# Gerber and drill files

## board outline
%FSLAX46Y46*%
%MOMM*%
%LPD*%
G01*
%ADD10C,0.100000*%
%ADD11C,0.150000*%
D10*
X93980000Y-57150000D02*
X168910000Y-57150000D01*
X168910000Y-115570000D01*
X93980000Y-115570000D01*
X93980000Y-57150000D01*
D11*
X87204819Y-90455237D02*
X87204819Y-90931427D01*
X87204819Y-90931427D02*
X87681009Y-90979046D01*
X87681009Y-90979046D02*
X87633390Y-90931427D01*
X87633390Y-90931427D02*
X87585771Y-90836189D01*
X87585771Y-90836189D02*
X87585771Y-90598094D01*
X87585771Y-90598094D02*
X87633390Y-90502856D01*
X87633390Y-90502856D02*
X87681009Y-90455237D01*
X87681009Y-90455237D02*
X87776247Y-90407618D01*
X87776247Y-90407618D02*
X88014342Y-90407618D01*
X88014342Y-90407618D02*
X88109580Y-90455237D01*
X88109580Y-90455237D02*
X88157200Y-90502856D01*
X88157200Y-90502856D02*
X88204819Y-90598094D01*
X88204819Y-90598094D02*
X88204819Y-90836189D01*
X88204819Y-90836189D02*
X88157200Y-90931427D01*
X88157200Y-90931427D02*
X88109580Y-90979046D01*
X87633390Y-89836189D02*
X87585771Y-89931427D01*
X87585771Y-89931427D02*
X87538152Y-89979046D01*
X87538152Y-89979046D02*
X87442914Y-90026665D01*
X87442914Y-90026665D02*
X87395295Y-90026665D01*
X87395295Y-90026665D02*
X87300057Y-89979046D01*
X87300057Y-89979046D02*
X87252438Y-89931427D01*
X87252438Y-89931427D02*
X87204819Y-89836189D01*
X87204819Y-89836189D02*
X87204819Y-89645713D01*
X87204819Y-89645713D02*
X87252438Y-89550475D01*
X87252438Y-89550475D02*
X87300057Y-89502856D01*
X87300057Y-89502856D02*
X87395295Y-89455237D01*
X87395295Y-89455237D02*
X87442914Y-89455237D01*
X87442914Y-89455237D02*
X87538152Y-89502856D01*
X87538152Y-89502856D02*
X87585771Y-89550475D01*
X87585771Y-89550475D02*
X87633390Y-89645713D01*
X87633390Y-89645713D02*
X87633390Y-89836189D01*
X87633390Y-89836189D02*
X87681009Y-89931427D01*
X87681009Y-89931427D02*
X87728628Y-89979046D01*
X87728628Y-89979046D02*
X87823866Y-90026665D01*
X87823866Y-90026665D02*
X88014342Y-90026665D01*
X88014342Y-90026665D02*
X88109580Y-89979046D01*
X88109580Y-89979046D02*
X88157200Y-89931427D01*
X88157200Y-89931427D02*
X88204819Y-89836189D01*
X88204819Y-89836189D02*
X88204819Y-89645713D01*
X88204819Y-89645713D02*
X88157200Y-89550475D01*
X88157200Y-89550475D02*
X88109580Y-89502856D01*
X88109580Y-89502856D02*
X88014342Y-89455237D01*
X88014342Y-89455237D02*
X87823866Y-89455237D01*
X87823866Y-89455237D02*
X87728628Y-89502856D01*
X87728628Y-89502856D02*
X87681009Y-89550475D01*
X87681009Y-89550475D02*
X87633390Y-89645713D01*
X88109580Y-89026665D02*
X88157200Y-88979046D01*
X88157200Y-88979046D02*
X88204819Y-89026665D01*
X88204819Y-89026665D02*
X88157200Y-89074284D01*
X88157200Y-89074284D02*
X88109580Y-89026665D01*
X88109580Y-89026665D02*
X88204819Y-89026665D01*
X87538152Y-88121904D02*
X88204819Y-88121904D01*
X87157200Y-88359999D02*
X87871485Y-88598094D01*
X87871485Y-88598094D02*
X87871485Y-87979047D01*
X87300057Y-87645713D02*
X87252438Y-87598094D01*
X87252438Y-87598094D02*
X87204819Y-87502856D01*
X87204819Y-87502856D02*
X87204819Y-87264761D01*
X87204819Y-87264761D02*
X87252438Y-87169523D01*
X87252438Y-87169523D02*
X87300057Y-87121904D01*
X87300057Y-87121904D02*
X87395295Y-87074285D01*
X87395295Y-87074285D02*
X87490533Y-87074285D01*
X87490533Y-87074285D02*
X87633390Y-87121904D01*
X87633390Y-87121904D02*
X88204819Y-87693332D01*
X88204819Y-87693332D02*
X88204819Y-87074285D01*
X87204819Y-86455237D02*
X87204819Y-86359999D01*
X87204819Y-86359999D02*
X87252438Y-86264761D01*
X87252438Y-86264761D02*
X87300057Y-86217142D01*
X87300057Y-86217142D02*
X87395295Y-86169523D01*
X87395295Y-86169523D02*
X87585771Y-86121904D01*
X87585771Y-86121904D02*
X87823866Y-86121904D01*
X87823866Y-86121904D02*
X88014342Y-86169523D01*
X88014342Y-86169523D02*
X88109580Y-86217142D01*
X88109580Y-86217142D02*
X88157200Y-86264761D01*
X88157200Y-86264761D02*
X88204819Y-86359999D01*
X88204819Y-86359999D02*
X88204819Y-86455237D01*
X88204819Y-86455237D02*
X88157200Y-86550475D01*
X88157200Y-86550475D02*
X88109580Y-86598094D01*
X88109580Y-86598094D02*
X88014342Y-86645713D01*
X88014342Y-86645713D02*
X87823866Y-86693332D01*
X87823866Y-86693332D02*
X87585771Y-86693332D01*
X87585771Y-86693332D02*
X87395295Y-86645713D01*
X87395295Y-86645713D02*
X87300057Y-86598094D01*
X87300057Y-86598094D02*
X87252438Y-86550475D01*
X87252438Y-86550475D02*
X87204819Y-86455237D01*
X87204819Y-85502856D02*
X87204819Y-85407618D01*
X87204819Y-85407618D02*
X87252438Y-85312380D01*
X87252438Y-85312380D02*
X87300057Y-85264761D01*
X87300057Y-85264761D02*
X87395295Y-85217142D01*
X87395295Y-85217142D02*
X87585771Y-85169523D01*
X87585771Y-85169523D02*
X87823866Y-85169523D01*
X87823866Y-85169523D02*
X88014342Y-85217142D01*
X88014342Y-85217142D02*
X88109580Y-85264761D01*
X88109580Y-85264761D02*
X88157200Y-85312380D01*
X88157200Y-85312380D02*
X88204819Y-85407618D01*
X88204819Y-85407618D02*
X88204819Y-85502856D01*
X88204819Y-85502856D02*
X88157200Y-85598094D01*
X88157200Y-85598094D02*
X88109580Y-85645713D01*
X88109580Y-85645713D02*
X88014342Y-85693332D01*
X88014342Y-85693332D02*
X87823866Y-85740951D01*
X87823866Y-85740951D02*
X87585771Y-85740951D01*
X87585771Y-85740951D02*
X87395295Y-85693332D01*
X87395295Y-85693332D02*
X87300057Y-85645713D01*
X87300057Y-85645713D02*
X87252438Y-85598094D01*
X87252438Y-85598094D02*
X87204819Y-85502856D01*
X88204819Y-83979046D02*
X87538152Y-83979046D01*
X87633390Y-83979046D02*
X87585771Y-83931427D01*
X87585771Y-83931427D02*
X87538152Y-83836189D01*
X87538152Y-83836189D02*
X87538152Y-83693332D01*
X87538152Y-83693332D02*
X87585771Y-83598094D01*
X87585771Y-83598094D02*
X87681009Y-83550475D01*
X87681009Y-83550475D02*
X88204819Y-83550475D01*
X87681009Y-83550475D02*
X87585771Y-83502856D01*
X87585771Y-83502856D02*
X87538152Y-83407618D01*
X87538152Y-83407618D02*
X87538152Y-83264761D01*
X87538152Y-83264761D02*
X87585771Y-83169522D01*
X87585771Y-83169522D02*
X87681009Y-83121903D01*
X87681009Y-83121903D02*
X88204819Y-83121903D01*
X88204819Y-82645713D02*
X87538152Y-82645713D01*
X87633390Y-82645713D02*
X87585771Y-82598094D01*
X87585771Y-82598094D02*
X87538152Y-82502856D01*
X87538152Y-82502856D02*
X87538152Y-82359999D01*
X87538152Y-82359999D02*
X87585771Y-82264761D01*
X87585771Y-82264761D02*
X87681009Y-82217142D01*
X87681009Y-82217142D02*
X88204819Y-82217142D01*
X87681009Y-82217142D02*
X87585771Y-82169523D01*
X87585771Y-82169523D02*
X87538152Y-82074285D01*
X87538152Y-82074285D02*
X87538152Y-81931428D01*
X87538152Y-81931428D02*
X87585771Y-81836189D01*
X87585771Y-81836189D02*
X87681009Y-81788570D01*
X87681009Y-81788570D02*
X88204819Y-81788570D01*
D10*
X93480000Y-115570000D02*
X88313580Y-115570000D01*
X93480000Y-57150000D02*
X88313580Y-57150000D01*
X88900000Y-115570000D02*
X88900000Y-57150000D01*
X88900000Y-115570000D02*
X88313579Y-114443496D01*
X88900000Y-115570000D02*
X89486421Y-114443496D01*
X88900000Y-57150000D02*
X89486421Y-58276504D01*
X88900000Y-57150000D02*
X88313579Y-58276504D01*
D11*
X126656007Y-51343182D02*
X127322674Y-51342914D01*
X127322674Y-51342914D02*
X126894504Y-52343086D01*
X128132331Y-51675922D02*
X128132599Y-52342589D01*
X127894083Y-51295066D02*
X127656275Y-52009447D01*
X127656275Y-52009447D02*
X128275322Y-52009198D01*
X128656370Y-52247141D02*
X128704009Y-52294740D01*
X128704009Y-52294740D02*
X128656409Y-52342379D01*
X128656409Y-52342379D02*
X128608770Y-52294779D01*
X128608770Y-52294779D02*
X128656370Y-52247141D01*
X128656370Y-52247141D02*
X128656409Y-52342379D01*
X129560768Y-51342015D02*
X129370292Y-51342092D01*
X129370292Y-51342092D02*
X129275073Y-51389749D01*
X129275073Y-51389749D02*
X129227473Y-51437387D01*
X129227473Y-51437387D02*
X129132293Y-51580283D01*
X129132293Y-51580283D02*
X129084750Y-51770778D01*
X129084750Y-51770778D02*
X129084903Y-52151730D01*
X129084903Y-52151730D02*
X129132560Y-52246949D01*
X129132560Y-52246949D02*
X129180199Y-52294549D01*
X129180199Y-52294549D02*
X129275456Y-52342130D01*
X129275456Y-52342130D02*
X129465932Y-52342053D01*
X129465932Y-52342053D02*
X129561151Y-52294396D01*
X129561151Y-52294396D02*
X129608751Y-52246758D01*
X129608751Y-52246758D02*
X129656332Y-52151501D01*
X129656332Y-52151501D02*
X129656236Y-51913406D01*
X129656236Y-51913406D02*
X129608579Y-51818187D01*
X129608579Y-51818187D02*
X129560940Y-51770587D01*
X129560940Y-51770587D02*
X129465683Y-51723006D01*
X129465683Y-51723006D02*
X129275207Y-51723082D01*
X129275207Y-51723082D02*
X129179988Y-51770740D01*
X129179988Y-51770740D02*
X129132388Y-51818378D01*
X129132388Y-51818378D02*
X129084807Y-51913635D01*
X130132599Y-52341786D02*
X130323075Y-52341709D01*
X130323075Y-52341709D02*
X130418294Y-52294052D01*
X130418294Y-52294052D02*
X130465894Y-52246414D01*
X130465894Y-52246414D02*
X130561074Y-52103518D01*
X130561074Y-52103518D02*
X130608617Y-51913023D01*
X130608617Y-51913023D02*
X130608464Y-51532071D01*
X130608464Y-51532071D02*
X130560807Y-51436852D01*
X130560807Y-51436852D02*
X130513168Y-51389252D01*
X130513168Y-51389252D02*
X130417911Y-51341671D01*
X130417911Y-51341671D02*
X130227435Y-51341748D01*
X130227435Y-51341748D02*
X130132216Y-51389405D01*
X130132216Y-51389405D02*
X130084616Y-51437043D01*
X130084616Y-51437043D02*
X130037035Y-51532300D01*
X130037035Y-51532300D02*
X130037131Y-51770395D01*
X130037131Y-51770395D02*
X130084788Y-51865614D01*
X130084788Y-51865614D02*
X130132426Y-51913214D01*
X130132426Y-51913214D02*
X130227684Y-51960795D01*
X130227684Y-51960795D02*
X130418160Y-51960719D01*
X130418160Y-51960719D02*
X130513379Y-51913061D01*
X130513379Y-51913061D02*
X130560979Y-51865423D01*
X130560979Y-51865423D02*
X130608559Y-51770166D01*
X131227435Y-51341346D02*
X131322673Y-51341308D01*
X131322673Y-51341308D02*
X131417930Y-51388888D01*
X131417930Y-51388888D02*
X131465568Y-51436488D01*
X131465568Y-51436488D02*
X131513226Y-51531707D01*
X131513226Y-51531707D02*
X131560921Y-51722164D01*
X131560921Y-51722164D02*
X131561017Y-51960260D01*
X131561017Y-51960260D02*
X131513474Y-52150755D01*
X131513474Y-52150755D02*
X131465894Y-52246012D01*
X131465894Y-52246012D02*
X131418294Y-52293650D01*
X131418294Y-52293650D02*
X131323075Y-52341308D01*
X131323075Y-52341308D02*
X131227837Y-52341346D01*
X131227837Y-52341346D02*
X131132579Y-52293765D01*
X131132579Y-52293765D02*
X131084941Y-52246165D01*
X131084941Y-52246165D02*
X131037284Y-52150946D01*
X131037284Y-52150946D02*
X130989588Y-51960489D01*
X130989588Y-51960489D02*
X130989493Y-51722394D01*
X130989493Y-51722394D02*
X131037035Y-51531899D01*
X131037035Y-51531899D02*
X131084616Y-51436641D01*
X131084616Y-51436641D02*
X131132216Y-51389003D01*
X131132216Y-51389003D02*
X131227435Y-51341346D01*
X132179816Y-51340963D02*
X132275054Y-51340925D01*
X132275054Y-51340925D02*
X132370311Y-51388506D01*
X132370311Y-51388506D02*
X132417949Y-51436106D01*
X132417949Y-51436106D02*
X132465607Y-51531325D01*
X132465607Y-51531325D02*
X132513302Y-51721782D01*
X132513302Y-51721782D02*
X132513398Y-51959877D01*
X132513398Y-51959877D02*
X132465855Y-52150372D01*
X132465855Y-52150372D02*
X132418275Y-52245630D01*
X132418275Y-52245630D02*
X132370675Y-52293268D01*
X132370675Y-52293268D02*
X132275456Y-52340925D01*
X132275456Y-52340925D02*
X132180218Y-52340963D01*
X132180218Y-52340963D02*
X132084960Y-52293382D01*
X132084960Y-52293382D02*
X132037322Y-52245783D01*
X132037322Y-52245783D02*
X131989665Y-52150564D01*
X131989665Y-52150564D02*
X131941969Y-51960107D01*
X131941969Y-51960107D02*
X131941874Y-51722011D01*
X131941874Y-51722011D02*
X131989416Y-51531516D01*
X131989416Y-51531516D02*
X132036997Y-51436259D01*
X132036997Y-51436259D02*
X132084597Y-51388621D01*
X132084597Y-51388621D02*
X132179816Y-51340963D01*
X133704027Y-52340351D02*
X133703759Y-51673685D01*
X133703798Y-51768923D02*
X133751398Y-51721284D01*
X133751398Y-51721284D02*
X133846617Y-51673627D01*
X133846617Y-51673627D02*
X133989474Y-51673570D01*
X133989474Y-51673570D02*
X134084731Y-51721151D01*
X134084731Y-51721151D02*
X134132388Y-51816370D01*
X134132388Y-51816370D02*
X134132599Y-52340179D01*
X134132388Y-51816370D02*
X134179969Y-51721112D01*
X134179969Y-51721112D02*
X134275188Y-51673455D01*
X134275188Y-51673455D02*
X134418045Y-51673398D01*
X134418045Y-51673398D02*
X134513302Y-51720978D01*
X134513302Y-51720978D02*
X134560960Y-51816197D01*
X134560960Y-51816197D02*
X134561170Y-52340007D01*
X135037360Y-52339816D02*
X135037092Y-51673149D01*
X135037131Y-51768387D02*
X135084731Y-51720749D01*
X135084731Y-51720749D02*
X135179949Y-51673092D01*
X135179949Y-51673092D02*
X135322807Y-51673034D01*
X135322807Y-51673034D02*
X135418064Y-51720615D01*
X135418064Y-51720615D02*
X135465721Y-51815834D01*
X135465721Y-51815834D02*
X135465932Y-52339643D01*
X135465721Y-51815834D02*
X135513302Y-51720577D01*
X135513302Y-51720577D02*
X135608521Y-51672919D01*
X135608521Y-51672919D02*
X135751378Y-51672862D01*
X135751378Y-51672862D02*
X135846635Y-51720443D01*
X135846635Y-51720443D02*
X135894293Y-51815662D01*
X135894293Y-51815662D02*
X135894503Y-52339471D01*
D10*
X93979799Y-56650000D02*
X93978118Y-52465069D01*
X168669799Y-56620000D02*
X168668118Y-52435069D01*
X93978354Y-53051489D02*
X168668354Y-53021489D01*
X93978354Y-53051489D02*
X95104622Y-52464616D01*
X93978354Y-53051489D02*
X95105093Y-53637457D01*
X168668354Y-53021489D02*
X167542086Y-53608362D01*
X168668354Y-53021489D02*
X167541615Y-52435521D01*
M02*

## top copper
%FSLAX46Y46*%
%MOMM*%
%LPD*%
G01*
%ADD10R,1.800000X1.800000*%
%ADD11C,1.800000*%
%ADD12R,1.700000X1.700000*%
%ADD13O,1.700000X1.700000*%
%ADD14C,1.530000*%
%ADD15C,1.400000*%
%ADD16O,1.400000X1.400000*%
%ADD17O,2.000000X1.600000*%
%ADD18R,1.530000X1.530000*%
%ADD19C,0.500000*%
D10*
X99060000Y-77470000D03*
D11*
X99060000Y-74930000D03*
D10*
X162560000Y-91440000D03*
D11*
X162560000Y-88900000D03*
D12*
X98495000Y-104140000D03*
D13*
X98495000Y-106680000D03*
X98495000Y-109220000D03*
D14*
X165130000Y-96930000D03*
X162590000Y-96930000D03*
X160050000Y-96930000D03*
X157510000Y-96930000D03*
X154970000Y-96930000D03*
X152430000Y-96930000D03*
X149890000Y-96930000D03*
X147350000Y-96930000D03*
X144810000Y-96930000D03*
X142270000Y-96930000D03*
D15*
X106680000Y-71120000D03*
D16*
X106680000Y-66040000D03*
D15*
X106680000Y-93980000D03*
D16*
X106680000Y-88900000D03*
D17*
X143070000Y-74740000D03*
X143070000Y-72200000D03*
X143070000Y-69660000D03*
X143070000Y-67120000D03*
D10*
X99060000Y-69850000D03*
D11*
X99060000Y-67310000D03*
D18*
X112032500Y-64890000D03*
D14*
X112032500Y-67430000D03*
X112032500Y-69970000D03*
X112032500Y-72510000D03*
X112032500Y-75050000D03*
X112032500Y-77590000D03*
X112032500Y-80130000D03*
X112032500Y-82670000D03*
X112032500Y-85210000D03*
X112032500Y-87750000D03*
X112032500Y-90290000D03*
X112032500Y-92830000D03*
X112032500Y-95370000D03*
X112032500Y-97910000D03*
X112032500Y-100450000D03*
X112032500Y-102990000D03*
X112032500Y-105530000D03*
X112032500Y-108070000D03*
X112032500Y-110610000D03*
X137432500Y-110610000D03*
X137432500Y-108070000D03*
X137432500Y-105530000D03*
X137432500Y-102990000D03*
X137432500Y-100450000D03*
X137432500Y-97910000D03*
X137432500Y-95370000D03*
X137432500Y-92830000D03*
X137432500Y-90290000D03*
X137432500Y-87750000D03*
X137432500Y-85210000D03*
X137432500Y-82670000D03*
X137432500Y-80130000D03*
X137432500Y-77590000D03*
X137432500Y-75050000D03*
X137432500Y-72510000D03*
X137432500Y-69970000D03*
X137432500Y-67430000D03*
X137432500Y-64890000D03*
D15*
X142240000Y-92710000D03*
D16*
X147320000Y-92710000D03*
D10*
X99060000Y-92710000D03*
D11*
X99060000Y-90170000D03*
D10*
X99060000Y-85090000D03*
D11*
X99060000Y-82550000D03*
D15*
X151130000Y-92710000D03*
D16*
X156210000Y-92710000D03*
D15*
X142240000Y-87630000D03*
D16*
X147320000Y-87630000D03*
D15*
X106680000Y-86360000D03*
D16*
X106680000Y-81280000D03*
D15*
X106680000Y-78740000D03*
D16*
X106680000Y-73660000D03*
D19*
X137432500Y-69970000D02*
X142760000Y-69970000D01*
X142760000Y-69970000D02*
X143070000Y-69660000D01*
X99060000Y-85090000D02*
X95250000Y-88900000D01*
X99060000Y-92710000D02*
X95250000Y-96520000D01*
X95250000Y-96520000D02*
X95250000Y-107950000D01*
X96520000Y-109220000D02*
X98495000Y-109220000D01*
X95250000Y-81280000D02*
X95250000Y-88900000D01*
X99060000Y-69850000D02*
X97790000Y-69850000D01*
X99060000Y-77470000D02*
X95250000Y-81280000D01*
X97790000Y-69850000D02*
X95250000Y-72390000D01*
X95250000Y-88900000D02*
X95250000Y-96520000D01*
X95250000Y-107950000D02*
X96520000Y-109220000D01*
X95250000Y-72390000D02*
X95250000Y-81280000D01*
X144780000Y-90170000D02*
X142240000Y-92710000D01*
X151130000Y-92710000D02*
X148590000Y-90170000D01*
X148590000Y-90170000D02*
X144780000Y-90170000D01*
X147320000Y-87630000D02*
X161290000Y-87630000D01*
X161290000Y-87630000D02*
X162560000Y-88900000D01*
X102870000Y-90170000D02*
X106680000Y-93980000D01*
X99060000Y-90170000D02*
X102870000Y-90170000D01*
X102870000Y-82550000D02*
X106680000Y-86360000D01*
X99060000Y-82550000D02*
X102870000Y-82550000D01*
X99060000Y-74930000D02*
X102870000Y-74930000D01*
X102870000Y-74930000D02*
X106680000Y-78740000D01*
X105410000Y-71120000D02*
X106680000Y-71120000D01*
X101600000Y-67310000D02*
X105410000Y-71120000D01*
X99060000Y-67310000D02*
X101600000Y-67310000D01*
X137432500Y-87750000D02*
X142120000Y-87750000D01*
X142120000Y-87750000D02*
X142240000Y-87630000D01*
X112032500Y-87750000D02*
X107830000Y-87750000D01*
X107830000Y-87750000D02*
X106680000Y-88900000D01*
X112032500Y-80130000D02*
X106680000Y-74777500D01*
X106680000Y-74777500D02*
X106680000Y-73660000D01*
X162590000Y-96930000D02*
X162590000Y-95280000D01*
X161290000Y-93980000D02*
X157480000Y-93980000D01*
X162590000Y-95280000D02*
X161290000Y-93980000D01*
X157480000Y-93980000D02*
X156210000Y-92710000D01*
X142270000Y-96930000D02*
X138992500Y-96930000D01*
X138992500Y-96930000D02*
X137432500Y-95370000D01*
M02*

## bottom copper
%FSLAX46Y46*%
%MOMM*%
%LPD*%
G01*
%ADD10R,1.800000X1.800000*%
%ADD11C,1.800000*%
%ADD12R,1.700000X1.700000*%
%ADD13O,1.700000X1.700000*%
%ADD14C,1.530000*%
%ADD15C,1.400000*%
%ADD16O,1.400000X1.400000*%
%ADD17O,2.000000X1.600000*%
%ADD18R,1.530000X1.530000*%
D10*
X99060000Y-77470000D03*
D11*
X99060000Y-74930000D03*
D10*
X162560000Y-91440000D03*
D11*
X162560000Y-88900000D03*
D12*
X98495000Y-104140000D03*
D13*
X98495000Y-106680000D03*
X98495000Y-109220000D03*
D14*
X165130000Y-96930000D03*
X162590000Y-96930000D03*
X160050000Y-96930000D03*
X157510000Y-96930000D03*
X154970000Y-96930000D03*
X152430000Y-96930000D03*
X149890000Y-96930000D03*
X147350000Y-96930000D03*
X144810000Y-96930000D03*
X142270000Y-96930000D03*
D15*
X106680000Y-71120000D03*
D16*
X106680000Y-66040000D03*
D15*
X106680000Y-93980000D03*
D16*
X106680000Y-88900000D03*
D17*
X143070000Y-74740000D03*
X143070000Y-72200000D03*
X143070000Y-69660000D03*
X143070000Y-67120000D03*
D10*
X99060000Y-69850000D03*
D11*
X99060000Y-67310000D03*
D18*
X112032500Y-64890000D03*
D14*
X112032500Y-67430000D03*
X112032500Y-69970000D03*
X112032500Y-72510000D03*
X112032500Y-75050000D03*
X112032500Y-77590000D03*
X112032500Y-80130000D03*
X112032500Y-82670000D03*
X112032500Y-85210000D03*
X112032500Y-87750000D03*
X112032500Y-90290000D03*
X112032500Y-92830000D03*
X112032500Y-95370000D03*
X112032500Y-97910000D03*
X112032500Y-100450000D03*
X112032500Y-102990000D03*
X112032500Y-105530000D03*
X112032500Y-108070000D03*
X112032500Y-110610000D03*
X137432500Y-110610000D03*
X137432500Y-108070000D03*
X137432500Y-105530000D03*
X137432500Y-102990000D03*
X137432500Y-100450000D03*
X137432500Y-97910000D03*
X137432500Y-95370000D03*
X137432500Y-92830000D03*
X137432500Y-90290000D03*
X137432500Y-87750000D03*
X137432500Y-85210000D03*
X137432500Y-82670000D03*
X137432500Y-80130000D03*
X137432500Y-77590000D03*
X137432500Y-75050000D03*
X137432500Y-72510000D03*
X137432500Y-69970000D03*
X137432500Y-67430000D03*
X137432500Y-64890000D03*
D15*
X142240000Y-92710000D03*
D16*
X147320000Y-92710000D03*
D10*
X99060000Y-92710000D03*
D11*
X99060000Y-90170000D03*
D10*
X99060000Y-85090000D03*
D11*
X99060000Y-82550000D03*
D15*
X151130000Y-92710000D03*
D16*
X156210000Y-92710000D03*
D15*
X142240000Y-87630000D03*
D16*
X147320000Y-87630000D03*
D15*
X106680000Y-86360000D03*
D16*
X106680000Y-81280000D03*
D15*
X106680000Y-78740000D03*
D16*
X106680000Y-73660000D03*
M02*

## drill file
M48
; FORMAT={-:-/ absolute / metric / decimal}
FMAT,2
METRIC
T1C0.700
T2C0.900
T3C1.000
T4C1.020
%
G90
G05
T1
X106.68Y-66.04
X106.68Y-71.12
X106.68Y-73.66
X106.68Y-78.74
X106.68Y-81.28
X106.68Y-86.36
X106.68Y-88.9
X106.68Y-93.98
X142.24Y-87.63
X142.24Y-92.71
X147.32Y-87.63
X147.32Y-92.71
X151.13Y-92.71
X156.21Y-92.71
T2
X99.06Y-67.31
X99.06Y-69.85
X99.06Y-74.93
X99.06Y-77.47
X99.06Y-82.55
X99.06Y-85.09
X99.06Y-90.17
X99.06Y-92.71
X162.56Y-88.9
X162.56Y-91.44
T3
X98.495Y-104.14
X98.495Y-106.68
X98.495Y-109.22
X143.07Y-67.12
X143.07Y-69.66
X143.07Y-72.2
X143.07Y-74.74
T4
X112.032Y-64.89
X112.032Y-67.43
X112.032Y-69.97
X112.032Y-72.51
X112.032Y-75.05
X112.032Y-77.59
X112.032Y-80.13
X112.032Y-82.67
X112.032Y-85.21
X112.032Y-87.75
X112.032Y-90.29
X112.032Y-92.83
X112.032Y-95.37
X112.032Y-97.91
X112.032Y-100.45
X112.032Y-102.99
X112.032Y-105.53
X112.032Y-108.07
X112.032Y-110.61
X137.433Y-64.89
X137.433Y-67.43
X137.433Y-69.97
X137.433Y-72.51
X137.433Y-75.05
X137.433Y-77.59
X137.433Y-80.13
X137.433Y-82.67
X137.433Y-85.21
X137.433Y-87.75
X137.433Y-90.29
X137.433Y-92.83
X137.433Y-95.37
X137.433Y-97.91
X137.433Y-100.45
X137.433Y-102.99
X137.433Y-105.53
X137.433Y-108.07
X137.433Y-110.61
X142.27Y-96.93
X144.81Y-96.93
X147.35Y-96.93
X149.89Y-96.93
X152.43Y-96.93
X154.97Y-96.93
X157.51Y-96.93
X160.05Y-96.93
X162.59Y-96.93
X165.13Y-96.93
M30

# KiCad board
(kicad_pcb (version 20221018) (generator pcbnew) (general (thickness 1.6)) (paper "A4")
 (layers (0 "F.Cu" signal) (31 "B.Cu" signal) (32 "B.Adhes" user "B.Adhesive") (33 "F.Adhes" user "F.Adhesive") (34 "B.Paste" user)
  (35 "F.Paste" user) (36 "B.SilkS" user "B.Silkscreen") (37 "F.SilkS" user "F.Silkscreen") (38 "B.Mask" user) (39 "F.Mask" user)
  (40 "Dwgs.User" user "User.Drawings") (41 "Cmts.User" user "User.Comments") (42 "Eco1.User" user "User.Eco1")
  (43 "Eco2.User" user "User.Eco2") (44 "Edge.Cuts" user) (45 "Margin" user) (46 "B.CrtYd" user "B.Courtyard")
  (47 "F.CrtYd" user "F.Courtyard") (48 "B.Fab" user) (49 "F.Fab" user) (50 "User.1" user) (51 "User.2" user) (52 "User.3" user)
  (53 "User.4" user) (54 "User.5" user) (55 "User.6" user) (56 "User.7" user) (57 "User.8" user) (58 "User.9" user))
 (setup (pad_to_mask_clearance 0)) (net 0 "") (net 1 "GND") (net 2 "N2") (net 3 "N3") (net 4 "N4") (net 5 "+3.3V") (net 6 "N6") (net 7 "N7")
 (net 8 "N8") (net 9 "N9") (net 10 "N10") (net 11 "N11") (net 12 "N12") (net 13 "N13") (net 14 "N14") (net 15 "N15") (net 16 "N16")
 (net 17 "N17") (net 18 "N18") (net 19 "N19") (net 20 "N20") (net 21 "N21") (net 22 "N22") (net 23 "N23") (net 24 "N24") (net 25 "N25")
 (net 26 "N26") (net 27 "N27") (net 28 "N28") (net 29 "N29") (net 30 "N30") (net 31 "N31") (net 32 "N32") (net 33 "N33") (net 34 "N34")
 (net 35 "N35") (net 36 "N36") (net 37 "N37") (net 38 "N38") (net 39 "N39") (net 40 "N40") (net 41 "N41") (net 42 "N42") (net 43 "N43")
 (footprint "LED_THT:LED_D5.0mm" (layer "F.Cu") (at 99.06 77.47 90)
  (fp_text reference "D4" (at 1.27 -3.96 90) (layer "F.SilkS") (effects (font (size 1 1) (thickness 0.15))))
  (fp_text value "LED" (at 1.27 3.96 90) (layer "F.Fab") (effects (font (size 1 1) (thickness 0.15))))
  (pad "1" thru_hole rect (at 0 0 90) (size 1.8 1.8) (drill 0.9) (layers "*.Cu" "*.Mask") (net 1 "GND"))
  (pad "2" thru_hole circle (at 2.54 0 90) (size 1.8 1.8) (drill 0.9) (layers "*.Cu" "*.Mask") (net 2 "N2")))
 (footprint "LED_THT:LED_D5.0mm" (layer "F.Cu") (at 162.56 91.44 90)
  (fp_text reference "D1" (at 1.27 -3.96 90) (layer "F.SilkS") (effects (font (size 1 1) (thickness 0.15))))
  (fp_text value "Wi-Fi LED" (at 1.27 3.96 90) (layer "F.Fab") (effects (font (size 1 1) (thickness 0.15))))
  (pad "1" thru_hole rect (at 0 0 90) (size 1.8 1.8) (drill 0.9) (layers "*.Cu" "*.Mask") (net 1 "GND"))
  (pad "2" thru_hole circle (at 2.54 0 90) (size 1.8 1.8) (drill 0.9) (layers "*.Cu" "*.Mask") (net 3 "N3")))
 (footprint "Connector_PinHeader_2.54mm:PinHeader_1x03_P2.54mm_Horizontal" (layer "F.Cu") (at 98.495 104.14)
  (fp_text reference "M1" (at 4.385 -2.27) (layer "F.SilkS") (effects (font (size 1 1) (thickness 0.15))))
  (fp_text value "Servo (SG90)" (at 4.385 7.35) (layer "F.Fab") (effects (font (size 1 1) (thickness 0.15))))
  (pad "1" thru_hole rect (at 0 0) (size 1.7 1.7) (drill 1) (layers "*.Cu" "*.Mask") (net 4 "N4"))
  (pad "2" thru_hole oval (at 0 2.54) (size 1.7 1.7) (drill 1) (layers "*.Cu" "*.Mask") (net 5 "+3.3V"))
  (pad "3" thru_hole oval (at 0 5.08) (size 1.7 1.7) (drill 1) (layers "*.Cu" "*.Mask") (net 1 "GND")))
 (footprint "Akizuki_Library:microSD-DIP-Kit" (layer "F.Cu") (at 153.7 95.66)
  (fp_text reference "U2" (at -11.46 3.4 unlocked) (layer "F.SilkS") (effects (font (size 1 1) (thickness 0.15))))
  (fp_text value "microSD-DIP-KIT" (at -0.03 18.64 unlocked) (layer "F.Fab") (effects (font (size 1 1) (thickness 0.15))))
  (pad "1" thru_hole circle (at 11.43 1.27) (size 1.53 1.53) (drill 1.02) (layers "*.Cu" "*.Mask") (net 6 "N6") (solder_mask_margin 0.102))
  (pad "2" thru_hole circle (at 8.89 1.27) (size 1.53 1.53) (drill 1.02) (layers "*.Cu" "*.Mask") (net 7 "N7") (solder_mask_margin 0.102))
  (pad "3" thru_hole circle (at 6.35 1.27) (size 1.53 1.53) (drill 1.02) (layers "*.Cu" "*.Mask") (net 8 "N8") (solder_mask_margin 0.102))
  (pad "4" thru_hole circle (at 3.81 1.27) (size 1.53 1.53) (drill 1.02) (layers "*.Cu" "*.Mask") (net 5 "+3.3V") (solder_mask_margin 0.102))
  (pad "5" thru_hole circle (at 1.27 1.27) (size 1.53 1.53) (drill 1.02) (layers "*.Cu" "*.Mask") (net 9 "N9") (solder_mask_margin 0.102))
  (pad "6" thru_hole circle (at -1.27 1.27) (size 1.53 1.53) (drill 1.02) (layers "*.Cu" "*.Mask") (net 1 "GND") (solder_mask_margin 0.102))
  (pad "7" thru_hole circle (at -3.81 1.27) (size 1.53 1.53) (drill 1.02) (layers "*.Cu" "*.Mask") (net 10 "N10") (solder_mask_margin 0.102))
  (pad "8" thru_hole circle (at -6.35 1.27) (size 1.53 1.53) (drill 1.02) (layers "*.Cu" "*.Mask") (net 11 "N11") (solder_mask_margin 0.102))
  (pad "9" thru_hole circle (at -8.89 1.27) (size 1.53 1.53) (drill 1.02) (layers "*.Cu" "*.Mask") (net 1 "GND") (solder_mask_margin 0.102))
  (pad "10" thru_hole circle (at -11.43 1.27) (size 1.53 1.53) (drill 1.02) (layers "*.Cu" "*.Mask") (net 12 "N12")
   (solder_mask_margin 0.102)))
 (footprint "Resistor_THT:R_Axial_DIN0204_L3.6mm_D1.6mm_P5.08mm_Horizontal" (layer "F.Cu") (at 106.68 71.12 90)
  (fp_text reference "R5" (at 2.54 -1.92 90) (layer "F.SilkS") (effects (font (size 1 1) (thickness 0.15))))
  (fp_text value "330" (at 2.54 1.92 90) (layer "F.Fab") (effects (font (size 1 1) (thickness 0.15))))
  (pad "1" thru_hole circle (at 0 0 90) (size 1.4 1.4) (drill 0.7) (layers "*.Cu" "*.Mask") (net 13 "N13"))
  (pad "2" thru_hole oval (at 5.08 0 90) (size 1.4 1.4) (drill 0.7) (layers "*.Cu" "*.Mask") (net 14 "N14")))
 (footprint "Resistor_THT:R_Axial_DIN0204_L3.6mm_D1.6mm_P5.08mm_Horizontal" (layer "F.Cu") (at 106.68 93.98 90)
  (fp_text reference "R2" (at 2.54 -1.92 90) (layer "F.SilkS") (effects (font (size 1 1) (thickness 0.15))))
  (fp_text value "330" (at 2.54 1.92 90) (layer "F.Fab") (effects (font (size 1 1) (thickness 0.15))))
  (pad "1" thru_hole circle (at 0 0 90) (size 1.4 1.4) (drill 0.7) (layers "*.Cu" "*.Mask") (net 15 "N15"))
  (pad "2" thru_hole oval (at 5.08 0 90) (size 1.4 1.4) (drill 0.7) (layers "*.Cu" "*.Mask") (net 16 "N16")))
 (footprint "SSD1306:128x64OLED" (layer "F.Cu") (at 153.67 71.12 90)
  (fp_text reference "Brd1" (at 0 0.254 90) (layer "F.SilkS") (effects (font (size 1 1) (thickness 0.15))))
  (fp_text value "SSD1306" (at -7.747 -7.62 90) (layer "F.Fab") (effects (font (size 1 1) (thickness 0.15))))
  (pad "1" thru_hole oval (at -3.62 -10.6 180) (size 2 1.6) (drill 1) (layers "*.Cu" "*.Mask") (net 1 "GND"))
  (pad "2" thru_hole oval (at -1.08 -10.6 180) (size 2 1.6) (drill 1) (layers "*.Cu" "*.Mask") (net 5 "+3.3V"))
  (pad "3" thru_hole oval (at 1.46 -10.6 180) (size 2 1.6) (drill 1) (layers "*.Cu" "*.Mask") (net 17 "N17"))
  (pad "4" thru_hole oval (at 4 -10.6 180) (size 2 1.6) (drill 1) (layers "*.Cu" "*.Mask") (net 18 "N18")))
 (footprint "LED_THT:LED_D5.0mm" (layer "F.Cu") (at 99.06 69.85 90)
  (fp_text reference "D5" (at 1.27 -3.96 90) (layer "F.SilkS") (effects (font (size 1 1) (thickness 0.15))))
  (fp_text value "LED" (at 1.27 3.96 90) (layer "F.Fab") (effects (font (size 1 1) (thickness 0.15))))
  (pad "1" thru_hole rect (at 0 0 90) (size 1.8 1.8) (drill 0.9) (layers "*.Cu" "*.Mask") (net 1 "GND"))
  (pad "2" thru_hole circle (at 2.54 0 90) (size 1.8 1.8) (drill 0.9) (layers "*.Cu" "*.Mask") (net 13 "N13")))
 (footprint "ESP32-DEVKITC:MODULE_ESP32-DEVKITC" (layer "F.Cu") (at 124.7325 87.74)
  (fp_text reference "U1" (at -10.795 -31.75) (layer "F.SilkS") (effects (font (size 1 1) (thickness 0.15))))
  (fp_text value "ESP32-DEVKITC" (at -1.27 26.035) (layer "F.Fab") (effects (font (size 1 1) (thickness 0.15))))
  (pad "1" thru_hole rect (at -12.7 -22.85) (size 1.53 1.53) (drill 1.02) (layers "*.Cu" "*.Mask") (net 5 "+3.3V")
   (solder_mask_margin 0.102))
  (pad "2" thru_hole circle (at -12.7 -20.31) (size 1.53 1.53) (drill 1.02) (layers "*.Cu" "*.Mask") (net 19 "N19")
   (solder_mask_margin 0.102))
  (pad "3" thru_hole circle (at -12.7 -17.77) (size 1.53 1.53) (drill 1.02) (layers "*.Cu" "*.Mask") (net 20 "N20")
   (solder_mask_margin 0.102))
  (pad "4" thru_hole circle (at -12.7 -15.23) (size 1.53 1.53) (drill 1.02) (layers "*.Cu" "*.Mask") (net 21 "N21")
   (solder_mask_margin 0.102))
  (pad "5" thru_hole circle (at -12.7 -12.69) (size 1.53 1.53) (drill 1.02) (layers "*.Cu" "*.Mask") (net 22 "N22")
   (solder_mask_margin 0.102))
  (pad "6" thru_hole circle (at -12.7 -10.15) (size 1.53 1.53) (drill 1.02) (layers "*.Cu" "*.Mask") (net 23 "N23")
   (solder_mask_margin 0.102))
  (pad "7" thru_hole circle (at -12.7 -7.61) (size 1.53 1.53) (drill 1.02) (layers "*.Cu" "*.Mask") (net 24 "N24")
   (solder_mask_margin 0.102))
  (pad "8" thru_hole circle (at -12.7 -5.07) (size 1.53 1.53) (drill 1.02) (layers "*.Cu" "*.Mask") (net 14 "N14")
   (solder_mask_margin 0.102))
  (pad "9" thru_hole circle (at -12.7 -2.53) (size 1.53 1.53) (drill 1.02) (layers "*.Cu" "*.Mask") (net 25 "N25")
   (solder_mask_margin 0.102))
  (pad "10" thru_hole circle (at -12.7 0.01) (size 1.53 1.53) (drill 1.02) (layers "*.Cu" "*.Mask") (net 16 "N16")
   (solder_mask_margin 0.102))
  (pad "11" thru_hole circle (at -12.7 2.55) (size 1.53 1.53) (drill 1.02) (layers "*.Cu" "*.Mask") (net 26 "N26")
   (solder_mask_margin 0.102))
  (pad "12" thru_hole circle (at -12.7 5.09) (size 1.53 1.53) (drill 1.02) (layers "*.Cu" "*.Mask") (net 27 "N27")
   (solder_mask_margin 0.102))
  (pad "13" thru_hole circle (at -12.7 7.63) (size 1.53 1.53) (drill 1.02) (layers "*.Cu" "*.Mask") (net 4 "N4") (solder_mask_margin 0.102))
  (pad "14" thru_hole circle (at -12.7 10.17) (size 1.53 1.53) (drill 1.02) (layers "*.Cu" "*.Mask") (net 1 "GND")
   (solder_mask_margin 0.102))
  (pad "15" thru_hole circle (at -12.7 12.71) (size 1.53 1.53) (drill 1.02) (layers "*.Cu" "*.Mask") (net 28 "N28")
   (solder_mask_margin 0.102))
  (pad "16" thru_hole circle (at -12.7 15.25) (size 1.53 1.53) (drill 1.02) (layers "*.Cu" "*.Mask") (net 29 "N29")
   (solder_mask_margin 0.102))
  (pad "17" thru_hole circle (at -12.7 17.79) (size 1.53 1.53) (drill 1.02) (layers "*.Cu" "*.Mask") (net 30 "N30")
   (solder_mask_margin 0.102))
  (pad "18" thru_hole circle (at -12.7 20.33) (size 1.53 1.53) (drill 1.02) (layers "*.Cu" "*.Mask") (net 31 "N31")
   (solder_mask_margin 0.102))
  (pad "19" thru_hole circle (at -12.7 22.87) (size 1.53 1.53) (drill 1.02) (layers "*.Cu" "*.Mask") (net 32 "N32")
   (solder_mask_margin 0.102))
  (pad "20" thru_hole circle (at 12.7 22.87) (size 1.53 1.53) (drill 1.02) (layers "*.Cu" "*.Mask") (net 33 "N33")
   (solder_mask_margin 0.102))
  (pad "21" thru_hole circle (at 12.7 20.33) (size 1.53 1.53) (drill 1.02) (layers "*.Cu" "*.Mask") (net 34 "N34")
   (solder_mask_margin 0.102))
  (pad "22" thru_hole circle (at 12.7 17.79) (size 1.53 1.53) (drill 1.02) (layers "*.Cu" "*.Mask") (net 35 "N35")
   (solder_mask_margin 0.102))
  (pad "23" thru_hole circle (at 12.7 15.25) (size 1.53 1.53) (drill 1.02) (layers "*.Cu" "*.Mask") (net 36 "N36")
   (solder_mask_margin 0.102))
  (pad "24" thru_hole circle (at 12.7 12.71) (size 1.53 1.53) (drill 1.02) (layers "*.Cu" "*.Mask") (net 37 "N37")
   (solder_mask_margin 0.102))
  (pad "25" thru_hole circle (at 12.7 10.17) (size 1.53 1.53) (drill 1.02) (layers "*.Cu" "*.Mask") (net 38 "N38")
   (solder_mask_margin 0.102))
  (pad "26" thru_hole circle (at 12.7 7.63) (size 1.53 1.53) (drill 1.02) (layers "*.Cu" "*.Mask") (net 12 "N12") (solder_mask_margin 0.102))
  (pad "27" thru_hole circle (at 12.7 5.09) (size 1.53 1.53) (drill 1.02) (layers "*.Cu" "*.Mask") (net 7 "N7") (solder_mask_margin 0.102))
  (pad "28" thru_hole circle (at 12.7 2.55) (size 1.53 1.53) (drill 1.02) (layers "*.Cu" "*.Mask") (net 8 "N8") (solder_mask_margin 0.102))
  (pad "29" thru_hole circle (at 12.7 0.01) (size 1.53 1.53) (drill 1.02) (layers "*.Cu" "*.Mask") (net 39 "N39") (solder_mask_margin 0.102))
  (pad "30" thru_hole circle (at 12.7 -2.53) (size 1.53 1.53) (drill 1.02) (layers "*.Cu" "*.Mask") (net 9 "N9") (solder_mask_margin 0.102))
  (pad "31" thru_hole circle (at 12.7 -5.07) (size 1.53 1.53) (drill 1.02) (layers "*.Cu" "*.Mask") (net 10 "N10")
   (solder_mask_margin 0.102))
  (pad "32" thru_hole circle (at 12.7 -7.61) (size 1.53 1.53) (drill 1.02) (layers "*.Cu" "*.Mask") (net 1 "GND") (solder_mask_margin 0.102))
  (pad "33" thru_hole circle (at 12.7 -10.15) (size 1.53 1.53) (drill 1.02) (layers "*.Cu" "*.Mask") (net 18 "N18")
   (solder_mask_margin 0.102))
  (pad "34" thru_hole circle (at 12.7 -12.69) (size 1.53 1.53) (drill 1.02) (layers "*.Cu" "*.Mask") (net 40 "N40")
   (solder_mask_margin 0.102))
  (pad "35" thru_hole circle (at 12.7 -15.23) (size 1.53 1.53) (drill 1.02) (layers "*.Cu" "*.Mask") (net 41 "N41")
   (solder_mask_margin 0.102))
  (pad "36" thru_hole circle (at 12.7 -17.77) (size 1.53 1.53) (drill 1.02) (layers "*.Cu" "*.Mask") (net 17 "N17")
   (solder_mask_margin 0.102))
  (pad "37" thru_hole circle (at 12.7 -20.31) (size 1.53 1.53) (drill 1.02) (layers "*.Cu" "*.Mask") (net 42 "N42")
   (solder_mask_margin 0.102))
  (pad "38" thru_hole circle (at 12.7 -22.85) (size 1.53 1.53) (drill 1.02) (layers "*.Cu" "*.Mask") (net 1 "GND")
   (solder_mask_margin 0.102)))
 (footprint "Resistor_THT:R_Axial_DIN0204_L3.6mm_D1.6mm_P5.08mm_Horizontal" (layer "F.Cu") (at 142.24 92.71)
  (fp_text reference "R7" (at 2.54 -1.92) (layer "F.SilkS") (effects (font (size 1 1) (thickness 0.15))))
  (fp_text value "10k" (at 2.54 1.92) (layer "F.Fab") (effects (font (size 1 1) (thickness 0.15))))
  (pad "1" thru_hole circle (at 0 0) (size 1.4 1.4) (drill 0.7) (layers "*.Cu" "*.Mask") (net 5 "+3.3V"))
  (pad "2" thru_hole oval (at 5.08 0) (size 1.4 1.4) (drill 0.7) (layers "*.Cu" "*.Mask") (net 9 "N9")))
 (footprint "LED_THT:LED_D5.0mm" (layer "F.Cu") (at 99.06 92.71 90)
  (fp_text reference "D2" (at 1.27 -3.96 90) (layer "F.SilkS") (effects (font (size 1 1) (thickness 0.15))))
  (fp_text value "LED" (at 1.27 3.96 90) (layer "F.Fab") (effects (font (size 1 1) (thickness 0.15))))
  (pad "1" thru_hole rect (at 0 0 90) (size 1.8 1.8) (drill 0.9) (layers "*.Cu" "*.Mask") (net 1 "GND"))
  (pad "2" thru_hole circle (at 2.54 0 90) (size 1.8 1.8) (drill 0.9) (layers "*.Cu" "*.Mask") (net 15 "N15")))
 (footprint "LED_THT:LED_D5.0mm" (layer "F.Cu") (at 99.06 85.09 90)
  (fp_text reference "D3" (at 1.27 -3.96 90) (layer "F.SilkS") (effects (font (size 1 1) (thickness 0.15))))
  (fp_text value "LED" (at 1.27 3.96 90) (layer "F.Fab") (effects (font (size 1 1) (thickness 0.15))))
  (pad "1" thru_hole rect (at 0 0 90) (size 1.8 1.8) (drill 0.9) (layers "*.Cu" "*.Mask") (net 1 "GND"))
  (pad "2" thru_hole circle (at 2.54 0 90) (size 1.8 1.8) (drill 0.9) (layers "*.Cu" "*.Mask") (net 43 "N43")))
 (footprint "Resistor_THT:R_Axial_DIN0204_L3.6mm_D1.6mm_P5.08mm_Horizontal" (layer "F.Cu") (at 151.13 92.71)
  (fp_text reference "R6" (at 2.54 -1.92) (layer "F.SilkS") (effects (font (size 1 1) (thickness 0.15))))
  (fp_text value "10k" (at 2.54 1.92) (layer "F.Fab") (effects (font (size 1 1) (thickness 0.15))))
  (pad "1" thru_hole circle (at 0 0) (size 1.4 1.4) (drill 0.7) (layers "*.Cu" "*.Mask") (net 5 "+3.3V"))
  (pad "2" thru_hole oval (at 5.08 0) (size 1.4 1.4) (drill 0.7) (layers "*.Cu" "*.Mask") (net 7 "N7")))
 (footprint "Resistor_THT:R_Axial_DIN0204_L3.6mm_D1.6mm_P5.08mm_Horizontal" (layer "F.Cu") (at 142.24 87.63)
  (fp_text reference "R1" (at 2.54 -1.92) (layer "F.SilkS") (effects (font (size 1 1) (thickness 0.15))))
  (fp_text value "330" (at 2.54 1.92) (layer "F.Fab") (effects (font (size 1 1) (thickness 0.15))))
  (pad "1" thru_hole circle (at 0 0) (size 1.4 1.4) (drill 0.7) (layers "*.Cu" "*.Mask") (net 39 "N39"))
  (pad "2" thru_hole oval (at 5.08 0) (size 1.4 1.4) (drill 0.7) (layers "*.Cu" "*.Mask") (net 3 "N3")))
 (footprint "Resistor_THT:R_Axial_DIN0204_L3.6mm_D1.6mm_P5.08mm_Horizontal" (layer "F.Cu") (at 106.68 86.36 90)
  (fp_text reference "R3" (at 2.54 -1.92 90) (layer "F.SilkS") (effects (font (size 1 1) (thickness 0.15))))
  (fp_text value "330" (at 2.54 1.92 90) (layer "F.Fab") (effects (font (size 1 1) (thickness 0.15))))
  (pad "1" thru_hole circle (at 0 0 90) (size 1.4 1.4) (drill 0.7) (layers "*.Cu" "*.Mask") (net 43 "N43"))
  (pad "2" thru_hole oval (at 5.08 0 90) (size 1.4 1.4) (drill 0.7) (layers "*.Cu" "*.Mask") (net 26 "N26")))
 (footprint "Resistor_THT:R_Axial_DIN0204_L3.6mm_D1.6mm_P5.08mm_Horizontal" (layer "F.Cu") (at 106.68 78.74 90)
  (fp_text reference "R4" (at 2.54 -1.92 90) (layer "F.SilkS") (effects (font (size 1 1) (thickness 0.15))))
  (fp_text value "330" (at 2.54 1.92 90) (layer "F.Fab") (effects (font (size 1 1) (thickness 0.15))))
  (pad "1" thru_hole circle (at 0 0 90) (size 1.4 1.4) (drill 0.7) (layers "*.Cu" "*.Mask") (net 2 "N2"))
  (pad "2" thru_hole oval (at 5.08 0 90) (size 1.4 1.4) (drill 0.7) (layers "*.Cu" "*.Mask") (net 24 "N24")))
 (gr_rect (start 93.98 57.15) (end 168.91 115.57) (stroke (width 0.1) (type default)) (fill none) (layer "Edge.Cuts"))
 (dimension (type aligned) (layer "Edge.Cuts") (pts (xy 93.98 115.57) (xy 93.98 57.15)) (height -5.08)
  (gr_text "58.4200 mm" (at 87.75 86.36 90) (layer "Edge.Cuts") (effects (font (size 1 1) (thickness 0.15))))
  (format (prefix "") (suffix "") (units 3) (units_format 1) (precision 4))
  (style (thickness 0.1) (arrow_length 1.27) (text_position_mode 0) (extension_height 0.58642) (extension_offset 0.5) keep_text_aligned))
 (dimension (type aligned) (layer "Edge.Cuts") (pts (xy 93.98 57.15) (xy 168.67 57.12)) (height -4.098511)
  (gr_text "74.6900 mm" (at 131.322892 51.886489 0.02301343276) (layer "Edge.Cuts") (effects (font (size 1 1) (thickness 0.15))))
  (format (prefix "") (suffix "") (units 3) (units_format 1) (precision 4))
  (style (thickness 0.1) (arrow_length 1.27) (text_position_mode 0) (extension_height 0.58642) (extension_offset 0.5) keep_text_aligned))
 (segment (start 137.4325 69.97) (end 142.76 69.97) (width 0.5) (layer "F.Cu") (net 17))
 (segment (start 142.76 69.97) (end 143.07 69.66) (width 0.5) (layer "F.Cu") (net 17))
 (segment (start 99.06 85.09) (end 95.25 88.9) (width 0.5) (layer "F.Cu") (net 1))
 (segment (start 99.06 92.71) (end 95.25 96.52) (width 0.5) (layer "F.Cu") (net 1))
 (segment (start 95.25 96.52) (end 95.25 107.95) (width 0.5) (layer "F.Cu") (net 1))
 (segment (start 96.52 109.22) (end 98.495 109.22) (width 0.5) (layer "F.Cu") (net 1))
 (segment (start 95.25 81.28) (end 95.25 88.9) (width 0.5) (layer "F.Cu") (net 1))
 (segment (start 99.06 69.85) (end 97.79 69.85) (width 0.5) (layer "F.Cu") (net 1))
 (segment (start 99.06 77.47) (end 95.25 81.28) (width 0.5) (layer "F.Cu") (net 1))
 (segment (start 97.79 69.85) (end 95.25 72.39) (width 0.5) (layer "F.Cu") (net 1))
 (segment (start 95.25 88.9) (end 95.25 96.52) (width 0.5) (layer "F.Cu") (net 1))
 (segment (start 95.25 107.95) (end 96.52 109.22) (width 0.5) (layer "F.Cu") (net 1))
 (segment (start 95.25 72.39) (end 95.25 81.28) (width 0.5) (layer "F.Cu") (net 1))
 (segment (start 144.78 90.17) (end 142.24 92.71) (width 0.5) (layer "F.Cu") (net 5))
 (segment (start 151.13 92.71) (end 148.59 90.17) (width 0.5) (layer "F.Cu") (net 5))
 (segment (start 148.59 90.17) (end 144.78 90.17) (width 0.5) (layer "F.Cu") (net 5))
 (segment (start 147.32 87.63) (end 161.29 87.63) (width 0.5) (layer "F.Cu") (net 3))
 (segment (start 161.29 87.63) (end 162.56 88.9) (width 0.5) (layer "F.Cu") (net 3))
 (segment (start 102.87 90.17) (end 106.68 93.98) (width 0.5) (layer "F.Cu") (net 15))
 (segment (start 99.06 90.17) (end 102.87 90.17) (width 0.5) (layer "F.Cu") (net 15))
 (segment (start 102.87 82.55) (end 106.68 86.36) (width 0.5) (layer "F.Cu") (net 43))
 (segment (start 99.06 82.55) (end 102.87 82.55) (width 0.5) (layer "F.Cu") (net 43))
 (segment (start 99.06 74.93) (end 102.87 74.93) (width 0.5) (layer "F.Cu") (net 2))
 (segment (start 102.87 74.93) (end 106.68 78.74) (width 0.5) (layer "F.Cu") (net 2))
 (segment (start 105.41 71.12) (end 106.68 71.12) (width 0.5) (layer "F.Cu") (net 13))
 (segment (start 101.6 67.31) (end 105.41 71.12) (width 0.5) (layer "F.Cu") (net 13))
 (segment (start 99.06 67.31) (end 101.6 67.31) (width 0.5) (layer "F.Cu") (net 13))
 (segment (start 137.4325 87.75) (end 142.12 87.75) (width 0.5) (layer "F.Cu") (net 39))
 (segment (start 142.12 87.75) (end 142.24 87.63) (width 0.5) (layer "F.Cu") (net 39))
 (segment (start 112.0325 87.75) (end 107.83 87.75) (width 0.5) (layer "F.Cu") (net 16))
 (segment (start 107.83 87.75) (end 106.68 88.9) (width 0.5) (layer "F.Cu") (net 16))
 (segment (start 112.0325 80.13) (end 106.68 74.7775) (width 0.5) (layer "F.Cu") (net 24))
 (segment (start 106.68 74.7775) (end 106.68 73.66) (width 0.5) (layer "F.Cu") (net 24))
 (segment (start 162.59 96.93) (end 162.59 95.28) (width 0.5) (layer "F.Cu") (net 7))
 (segment (start 161.29 93.98) (end 157.48 93.98) (width 0.5) (layer "F.Cu") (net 7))
 (segment (start 162.59 95.28) (end 161.29 93.98) (width 0.5) (layer "F.Cu") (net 7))
 (segment (start 157.48 93.98) (end 156.21 92.71) (width 0.5) (layer "F.Cu") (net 7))
 (segment (start 142.27 96.93) (end 138.9925 96.93) (width 0.5) (layer "F.Cu") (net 12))
 (segment (start 138.9925 96.93) (end 137.4325 95.37) (width 0.5) (layer "F.Cu") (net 12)))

